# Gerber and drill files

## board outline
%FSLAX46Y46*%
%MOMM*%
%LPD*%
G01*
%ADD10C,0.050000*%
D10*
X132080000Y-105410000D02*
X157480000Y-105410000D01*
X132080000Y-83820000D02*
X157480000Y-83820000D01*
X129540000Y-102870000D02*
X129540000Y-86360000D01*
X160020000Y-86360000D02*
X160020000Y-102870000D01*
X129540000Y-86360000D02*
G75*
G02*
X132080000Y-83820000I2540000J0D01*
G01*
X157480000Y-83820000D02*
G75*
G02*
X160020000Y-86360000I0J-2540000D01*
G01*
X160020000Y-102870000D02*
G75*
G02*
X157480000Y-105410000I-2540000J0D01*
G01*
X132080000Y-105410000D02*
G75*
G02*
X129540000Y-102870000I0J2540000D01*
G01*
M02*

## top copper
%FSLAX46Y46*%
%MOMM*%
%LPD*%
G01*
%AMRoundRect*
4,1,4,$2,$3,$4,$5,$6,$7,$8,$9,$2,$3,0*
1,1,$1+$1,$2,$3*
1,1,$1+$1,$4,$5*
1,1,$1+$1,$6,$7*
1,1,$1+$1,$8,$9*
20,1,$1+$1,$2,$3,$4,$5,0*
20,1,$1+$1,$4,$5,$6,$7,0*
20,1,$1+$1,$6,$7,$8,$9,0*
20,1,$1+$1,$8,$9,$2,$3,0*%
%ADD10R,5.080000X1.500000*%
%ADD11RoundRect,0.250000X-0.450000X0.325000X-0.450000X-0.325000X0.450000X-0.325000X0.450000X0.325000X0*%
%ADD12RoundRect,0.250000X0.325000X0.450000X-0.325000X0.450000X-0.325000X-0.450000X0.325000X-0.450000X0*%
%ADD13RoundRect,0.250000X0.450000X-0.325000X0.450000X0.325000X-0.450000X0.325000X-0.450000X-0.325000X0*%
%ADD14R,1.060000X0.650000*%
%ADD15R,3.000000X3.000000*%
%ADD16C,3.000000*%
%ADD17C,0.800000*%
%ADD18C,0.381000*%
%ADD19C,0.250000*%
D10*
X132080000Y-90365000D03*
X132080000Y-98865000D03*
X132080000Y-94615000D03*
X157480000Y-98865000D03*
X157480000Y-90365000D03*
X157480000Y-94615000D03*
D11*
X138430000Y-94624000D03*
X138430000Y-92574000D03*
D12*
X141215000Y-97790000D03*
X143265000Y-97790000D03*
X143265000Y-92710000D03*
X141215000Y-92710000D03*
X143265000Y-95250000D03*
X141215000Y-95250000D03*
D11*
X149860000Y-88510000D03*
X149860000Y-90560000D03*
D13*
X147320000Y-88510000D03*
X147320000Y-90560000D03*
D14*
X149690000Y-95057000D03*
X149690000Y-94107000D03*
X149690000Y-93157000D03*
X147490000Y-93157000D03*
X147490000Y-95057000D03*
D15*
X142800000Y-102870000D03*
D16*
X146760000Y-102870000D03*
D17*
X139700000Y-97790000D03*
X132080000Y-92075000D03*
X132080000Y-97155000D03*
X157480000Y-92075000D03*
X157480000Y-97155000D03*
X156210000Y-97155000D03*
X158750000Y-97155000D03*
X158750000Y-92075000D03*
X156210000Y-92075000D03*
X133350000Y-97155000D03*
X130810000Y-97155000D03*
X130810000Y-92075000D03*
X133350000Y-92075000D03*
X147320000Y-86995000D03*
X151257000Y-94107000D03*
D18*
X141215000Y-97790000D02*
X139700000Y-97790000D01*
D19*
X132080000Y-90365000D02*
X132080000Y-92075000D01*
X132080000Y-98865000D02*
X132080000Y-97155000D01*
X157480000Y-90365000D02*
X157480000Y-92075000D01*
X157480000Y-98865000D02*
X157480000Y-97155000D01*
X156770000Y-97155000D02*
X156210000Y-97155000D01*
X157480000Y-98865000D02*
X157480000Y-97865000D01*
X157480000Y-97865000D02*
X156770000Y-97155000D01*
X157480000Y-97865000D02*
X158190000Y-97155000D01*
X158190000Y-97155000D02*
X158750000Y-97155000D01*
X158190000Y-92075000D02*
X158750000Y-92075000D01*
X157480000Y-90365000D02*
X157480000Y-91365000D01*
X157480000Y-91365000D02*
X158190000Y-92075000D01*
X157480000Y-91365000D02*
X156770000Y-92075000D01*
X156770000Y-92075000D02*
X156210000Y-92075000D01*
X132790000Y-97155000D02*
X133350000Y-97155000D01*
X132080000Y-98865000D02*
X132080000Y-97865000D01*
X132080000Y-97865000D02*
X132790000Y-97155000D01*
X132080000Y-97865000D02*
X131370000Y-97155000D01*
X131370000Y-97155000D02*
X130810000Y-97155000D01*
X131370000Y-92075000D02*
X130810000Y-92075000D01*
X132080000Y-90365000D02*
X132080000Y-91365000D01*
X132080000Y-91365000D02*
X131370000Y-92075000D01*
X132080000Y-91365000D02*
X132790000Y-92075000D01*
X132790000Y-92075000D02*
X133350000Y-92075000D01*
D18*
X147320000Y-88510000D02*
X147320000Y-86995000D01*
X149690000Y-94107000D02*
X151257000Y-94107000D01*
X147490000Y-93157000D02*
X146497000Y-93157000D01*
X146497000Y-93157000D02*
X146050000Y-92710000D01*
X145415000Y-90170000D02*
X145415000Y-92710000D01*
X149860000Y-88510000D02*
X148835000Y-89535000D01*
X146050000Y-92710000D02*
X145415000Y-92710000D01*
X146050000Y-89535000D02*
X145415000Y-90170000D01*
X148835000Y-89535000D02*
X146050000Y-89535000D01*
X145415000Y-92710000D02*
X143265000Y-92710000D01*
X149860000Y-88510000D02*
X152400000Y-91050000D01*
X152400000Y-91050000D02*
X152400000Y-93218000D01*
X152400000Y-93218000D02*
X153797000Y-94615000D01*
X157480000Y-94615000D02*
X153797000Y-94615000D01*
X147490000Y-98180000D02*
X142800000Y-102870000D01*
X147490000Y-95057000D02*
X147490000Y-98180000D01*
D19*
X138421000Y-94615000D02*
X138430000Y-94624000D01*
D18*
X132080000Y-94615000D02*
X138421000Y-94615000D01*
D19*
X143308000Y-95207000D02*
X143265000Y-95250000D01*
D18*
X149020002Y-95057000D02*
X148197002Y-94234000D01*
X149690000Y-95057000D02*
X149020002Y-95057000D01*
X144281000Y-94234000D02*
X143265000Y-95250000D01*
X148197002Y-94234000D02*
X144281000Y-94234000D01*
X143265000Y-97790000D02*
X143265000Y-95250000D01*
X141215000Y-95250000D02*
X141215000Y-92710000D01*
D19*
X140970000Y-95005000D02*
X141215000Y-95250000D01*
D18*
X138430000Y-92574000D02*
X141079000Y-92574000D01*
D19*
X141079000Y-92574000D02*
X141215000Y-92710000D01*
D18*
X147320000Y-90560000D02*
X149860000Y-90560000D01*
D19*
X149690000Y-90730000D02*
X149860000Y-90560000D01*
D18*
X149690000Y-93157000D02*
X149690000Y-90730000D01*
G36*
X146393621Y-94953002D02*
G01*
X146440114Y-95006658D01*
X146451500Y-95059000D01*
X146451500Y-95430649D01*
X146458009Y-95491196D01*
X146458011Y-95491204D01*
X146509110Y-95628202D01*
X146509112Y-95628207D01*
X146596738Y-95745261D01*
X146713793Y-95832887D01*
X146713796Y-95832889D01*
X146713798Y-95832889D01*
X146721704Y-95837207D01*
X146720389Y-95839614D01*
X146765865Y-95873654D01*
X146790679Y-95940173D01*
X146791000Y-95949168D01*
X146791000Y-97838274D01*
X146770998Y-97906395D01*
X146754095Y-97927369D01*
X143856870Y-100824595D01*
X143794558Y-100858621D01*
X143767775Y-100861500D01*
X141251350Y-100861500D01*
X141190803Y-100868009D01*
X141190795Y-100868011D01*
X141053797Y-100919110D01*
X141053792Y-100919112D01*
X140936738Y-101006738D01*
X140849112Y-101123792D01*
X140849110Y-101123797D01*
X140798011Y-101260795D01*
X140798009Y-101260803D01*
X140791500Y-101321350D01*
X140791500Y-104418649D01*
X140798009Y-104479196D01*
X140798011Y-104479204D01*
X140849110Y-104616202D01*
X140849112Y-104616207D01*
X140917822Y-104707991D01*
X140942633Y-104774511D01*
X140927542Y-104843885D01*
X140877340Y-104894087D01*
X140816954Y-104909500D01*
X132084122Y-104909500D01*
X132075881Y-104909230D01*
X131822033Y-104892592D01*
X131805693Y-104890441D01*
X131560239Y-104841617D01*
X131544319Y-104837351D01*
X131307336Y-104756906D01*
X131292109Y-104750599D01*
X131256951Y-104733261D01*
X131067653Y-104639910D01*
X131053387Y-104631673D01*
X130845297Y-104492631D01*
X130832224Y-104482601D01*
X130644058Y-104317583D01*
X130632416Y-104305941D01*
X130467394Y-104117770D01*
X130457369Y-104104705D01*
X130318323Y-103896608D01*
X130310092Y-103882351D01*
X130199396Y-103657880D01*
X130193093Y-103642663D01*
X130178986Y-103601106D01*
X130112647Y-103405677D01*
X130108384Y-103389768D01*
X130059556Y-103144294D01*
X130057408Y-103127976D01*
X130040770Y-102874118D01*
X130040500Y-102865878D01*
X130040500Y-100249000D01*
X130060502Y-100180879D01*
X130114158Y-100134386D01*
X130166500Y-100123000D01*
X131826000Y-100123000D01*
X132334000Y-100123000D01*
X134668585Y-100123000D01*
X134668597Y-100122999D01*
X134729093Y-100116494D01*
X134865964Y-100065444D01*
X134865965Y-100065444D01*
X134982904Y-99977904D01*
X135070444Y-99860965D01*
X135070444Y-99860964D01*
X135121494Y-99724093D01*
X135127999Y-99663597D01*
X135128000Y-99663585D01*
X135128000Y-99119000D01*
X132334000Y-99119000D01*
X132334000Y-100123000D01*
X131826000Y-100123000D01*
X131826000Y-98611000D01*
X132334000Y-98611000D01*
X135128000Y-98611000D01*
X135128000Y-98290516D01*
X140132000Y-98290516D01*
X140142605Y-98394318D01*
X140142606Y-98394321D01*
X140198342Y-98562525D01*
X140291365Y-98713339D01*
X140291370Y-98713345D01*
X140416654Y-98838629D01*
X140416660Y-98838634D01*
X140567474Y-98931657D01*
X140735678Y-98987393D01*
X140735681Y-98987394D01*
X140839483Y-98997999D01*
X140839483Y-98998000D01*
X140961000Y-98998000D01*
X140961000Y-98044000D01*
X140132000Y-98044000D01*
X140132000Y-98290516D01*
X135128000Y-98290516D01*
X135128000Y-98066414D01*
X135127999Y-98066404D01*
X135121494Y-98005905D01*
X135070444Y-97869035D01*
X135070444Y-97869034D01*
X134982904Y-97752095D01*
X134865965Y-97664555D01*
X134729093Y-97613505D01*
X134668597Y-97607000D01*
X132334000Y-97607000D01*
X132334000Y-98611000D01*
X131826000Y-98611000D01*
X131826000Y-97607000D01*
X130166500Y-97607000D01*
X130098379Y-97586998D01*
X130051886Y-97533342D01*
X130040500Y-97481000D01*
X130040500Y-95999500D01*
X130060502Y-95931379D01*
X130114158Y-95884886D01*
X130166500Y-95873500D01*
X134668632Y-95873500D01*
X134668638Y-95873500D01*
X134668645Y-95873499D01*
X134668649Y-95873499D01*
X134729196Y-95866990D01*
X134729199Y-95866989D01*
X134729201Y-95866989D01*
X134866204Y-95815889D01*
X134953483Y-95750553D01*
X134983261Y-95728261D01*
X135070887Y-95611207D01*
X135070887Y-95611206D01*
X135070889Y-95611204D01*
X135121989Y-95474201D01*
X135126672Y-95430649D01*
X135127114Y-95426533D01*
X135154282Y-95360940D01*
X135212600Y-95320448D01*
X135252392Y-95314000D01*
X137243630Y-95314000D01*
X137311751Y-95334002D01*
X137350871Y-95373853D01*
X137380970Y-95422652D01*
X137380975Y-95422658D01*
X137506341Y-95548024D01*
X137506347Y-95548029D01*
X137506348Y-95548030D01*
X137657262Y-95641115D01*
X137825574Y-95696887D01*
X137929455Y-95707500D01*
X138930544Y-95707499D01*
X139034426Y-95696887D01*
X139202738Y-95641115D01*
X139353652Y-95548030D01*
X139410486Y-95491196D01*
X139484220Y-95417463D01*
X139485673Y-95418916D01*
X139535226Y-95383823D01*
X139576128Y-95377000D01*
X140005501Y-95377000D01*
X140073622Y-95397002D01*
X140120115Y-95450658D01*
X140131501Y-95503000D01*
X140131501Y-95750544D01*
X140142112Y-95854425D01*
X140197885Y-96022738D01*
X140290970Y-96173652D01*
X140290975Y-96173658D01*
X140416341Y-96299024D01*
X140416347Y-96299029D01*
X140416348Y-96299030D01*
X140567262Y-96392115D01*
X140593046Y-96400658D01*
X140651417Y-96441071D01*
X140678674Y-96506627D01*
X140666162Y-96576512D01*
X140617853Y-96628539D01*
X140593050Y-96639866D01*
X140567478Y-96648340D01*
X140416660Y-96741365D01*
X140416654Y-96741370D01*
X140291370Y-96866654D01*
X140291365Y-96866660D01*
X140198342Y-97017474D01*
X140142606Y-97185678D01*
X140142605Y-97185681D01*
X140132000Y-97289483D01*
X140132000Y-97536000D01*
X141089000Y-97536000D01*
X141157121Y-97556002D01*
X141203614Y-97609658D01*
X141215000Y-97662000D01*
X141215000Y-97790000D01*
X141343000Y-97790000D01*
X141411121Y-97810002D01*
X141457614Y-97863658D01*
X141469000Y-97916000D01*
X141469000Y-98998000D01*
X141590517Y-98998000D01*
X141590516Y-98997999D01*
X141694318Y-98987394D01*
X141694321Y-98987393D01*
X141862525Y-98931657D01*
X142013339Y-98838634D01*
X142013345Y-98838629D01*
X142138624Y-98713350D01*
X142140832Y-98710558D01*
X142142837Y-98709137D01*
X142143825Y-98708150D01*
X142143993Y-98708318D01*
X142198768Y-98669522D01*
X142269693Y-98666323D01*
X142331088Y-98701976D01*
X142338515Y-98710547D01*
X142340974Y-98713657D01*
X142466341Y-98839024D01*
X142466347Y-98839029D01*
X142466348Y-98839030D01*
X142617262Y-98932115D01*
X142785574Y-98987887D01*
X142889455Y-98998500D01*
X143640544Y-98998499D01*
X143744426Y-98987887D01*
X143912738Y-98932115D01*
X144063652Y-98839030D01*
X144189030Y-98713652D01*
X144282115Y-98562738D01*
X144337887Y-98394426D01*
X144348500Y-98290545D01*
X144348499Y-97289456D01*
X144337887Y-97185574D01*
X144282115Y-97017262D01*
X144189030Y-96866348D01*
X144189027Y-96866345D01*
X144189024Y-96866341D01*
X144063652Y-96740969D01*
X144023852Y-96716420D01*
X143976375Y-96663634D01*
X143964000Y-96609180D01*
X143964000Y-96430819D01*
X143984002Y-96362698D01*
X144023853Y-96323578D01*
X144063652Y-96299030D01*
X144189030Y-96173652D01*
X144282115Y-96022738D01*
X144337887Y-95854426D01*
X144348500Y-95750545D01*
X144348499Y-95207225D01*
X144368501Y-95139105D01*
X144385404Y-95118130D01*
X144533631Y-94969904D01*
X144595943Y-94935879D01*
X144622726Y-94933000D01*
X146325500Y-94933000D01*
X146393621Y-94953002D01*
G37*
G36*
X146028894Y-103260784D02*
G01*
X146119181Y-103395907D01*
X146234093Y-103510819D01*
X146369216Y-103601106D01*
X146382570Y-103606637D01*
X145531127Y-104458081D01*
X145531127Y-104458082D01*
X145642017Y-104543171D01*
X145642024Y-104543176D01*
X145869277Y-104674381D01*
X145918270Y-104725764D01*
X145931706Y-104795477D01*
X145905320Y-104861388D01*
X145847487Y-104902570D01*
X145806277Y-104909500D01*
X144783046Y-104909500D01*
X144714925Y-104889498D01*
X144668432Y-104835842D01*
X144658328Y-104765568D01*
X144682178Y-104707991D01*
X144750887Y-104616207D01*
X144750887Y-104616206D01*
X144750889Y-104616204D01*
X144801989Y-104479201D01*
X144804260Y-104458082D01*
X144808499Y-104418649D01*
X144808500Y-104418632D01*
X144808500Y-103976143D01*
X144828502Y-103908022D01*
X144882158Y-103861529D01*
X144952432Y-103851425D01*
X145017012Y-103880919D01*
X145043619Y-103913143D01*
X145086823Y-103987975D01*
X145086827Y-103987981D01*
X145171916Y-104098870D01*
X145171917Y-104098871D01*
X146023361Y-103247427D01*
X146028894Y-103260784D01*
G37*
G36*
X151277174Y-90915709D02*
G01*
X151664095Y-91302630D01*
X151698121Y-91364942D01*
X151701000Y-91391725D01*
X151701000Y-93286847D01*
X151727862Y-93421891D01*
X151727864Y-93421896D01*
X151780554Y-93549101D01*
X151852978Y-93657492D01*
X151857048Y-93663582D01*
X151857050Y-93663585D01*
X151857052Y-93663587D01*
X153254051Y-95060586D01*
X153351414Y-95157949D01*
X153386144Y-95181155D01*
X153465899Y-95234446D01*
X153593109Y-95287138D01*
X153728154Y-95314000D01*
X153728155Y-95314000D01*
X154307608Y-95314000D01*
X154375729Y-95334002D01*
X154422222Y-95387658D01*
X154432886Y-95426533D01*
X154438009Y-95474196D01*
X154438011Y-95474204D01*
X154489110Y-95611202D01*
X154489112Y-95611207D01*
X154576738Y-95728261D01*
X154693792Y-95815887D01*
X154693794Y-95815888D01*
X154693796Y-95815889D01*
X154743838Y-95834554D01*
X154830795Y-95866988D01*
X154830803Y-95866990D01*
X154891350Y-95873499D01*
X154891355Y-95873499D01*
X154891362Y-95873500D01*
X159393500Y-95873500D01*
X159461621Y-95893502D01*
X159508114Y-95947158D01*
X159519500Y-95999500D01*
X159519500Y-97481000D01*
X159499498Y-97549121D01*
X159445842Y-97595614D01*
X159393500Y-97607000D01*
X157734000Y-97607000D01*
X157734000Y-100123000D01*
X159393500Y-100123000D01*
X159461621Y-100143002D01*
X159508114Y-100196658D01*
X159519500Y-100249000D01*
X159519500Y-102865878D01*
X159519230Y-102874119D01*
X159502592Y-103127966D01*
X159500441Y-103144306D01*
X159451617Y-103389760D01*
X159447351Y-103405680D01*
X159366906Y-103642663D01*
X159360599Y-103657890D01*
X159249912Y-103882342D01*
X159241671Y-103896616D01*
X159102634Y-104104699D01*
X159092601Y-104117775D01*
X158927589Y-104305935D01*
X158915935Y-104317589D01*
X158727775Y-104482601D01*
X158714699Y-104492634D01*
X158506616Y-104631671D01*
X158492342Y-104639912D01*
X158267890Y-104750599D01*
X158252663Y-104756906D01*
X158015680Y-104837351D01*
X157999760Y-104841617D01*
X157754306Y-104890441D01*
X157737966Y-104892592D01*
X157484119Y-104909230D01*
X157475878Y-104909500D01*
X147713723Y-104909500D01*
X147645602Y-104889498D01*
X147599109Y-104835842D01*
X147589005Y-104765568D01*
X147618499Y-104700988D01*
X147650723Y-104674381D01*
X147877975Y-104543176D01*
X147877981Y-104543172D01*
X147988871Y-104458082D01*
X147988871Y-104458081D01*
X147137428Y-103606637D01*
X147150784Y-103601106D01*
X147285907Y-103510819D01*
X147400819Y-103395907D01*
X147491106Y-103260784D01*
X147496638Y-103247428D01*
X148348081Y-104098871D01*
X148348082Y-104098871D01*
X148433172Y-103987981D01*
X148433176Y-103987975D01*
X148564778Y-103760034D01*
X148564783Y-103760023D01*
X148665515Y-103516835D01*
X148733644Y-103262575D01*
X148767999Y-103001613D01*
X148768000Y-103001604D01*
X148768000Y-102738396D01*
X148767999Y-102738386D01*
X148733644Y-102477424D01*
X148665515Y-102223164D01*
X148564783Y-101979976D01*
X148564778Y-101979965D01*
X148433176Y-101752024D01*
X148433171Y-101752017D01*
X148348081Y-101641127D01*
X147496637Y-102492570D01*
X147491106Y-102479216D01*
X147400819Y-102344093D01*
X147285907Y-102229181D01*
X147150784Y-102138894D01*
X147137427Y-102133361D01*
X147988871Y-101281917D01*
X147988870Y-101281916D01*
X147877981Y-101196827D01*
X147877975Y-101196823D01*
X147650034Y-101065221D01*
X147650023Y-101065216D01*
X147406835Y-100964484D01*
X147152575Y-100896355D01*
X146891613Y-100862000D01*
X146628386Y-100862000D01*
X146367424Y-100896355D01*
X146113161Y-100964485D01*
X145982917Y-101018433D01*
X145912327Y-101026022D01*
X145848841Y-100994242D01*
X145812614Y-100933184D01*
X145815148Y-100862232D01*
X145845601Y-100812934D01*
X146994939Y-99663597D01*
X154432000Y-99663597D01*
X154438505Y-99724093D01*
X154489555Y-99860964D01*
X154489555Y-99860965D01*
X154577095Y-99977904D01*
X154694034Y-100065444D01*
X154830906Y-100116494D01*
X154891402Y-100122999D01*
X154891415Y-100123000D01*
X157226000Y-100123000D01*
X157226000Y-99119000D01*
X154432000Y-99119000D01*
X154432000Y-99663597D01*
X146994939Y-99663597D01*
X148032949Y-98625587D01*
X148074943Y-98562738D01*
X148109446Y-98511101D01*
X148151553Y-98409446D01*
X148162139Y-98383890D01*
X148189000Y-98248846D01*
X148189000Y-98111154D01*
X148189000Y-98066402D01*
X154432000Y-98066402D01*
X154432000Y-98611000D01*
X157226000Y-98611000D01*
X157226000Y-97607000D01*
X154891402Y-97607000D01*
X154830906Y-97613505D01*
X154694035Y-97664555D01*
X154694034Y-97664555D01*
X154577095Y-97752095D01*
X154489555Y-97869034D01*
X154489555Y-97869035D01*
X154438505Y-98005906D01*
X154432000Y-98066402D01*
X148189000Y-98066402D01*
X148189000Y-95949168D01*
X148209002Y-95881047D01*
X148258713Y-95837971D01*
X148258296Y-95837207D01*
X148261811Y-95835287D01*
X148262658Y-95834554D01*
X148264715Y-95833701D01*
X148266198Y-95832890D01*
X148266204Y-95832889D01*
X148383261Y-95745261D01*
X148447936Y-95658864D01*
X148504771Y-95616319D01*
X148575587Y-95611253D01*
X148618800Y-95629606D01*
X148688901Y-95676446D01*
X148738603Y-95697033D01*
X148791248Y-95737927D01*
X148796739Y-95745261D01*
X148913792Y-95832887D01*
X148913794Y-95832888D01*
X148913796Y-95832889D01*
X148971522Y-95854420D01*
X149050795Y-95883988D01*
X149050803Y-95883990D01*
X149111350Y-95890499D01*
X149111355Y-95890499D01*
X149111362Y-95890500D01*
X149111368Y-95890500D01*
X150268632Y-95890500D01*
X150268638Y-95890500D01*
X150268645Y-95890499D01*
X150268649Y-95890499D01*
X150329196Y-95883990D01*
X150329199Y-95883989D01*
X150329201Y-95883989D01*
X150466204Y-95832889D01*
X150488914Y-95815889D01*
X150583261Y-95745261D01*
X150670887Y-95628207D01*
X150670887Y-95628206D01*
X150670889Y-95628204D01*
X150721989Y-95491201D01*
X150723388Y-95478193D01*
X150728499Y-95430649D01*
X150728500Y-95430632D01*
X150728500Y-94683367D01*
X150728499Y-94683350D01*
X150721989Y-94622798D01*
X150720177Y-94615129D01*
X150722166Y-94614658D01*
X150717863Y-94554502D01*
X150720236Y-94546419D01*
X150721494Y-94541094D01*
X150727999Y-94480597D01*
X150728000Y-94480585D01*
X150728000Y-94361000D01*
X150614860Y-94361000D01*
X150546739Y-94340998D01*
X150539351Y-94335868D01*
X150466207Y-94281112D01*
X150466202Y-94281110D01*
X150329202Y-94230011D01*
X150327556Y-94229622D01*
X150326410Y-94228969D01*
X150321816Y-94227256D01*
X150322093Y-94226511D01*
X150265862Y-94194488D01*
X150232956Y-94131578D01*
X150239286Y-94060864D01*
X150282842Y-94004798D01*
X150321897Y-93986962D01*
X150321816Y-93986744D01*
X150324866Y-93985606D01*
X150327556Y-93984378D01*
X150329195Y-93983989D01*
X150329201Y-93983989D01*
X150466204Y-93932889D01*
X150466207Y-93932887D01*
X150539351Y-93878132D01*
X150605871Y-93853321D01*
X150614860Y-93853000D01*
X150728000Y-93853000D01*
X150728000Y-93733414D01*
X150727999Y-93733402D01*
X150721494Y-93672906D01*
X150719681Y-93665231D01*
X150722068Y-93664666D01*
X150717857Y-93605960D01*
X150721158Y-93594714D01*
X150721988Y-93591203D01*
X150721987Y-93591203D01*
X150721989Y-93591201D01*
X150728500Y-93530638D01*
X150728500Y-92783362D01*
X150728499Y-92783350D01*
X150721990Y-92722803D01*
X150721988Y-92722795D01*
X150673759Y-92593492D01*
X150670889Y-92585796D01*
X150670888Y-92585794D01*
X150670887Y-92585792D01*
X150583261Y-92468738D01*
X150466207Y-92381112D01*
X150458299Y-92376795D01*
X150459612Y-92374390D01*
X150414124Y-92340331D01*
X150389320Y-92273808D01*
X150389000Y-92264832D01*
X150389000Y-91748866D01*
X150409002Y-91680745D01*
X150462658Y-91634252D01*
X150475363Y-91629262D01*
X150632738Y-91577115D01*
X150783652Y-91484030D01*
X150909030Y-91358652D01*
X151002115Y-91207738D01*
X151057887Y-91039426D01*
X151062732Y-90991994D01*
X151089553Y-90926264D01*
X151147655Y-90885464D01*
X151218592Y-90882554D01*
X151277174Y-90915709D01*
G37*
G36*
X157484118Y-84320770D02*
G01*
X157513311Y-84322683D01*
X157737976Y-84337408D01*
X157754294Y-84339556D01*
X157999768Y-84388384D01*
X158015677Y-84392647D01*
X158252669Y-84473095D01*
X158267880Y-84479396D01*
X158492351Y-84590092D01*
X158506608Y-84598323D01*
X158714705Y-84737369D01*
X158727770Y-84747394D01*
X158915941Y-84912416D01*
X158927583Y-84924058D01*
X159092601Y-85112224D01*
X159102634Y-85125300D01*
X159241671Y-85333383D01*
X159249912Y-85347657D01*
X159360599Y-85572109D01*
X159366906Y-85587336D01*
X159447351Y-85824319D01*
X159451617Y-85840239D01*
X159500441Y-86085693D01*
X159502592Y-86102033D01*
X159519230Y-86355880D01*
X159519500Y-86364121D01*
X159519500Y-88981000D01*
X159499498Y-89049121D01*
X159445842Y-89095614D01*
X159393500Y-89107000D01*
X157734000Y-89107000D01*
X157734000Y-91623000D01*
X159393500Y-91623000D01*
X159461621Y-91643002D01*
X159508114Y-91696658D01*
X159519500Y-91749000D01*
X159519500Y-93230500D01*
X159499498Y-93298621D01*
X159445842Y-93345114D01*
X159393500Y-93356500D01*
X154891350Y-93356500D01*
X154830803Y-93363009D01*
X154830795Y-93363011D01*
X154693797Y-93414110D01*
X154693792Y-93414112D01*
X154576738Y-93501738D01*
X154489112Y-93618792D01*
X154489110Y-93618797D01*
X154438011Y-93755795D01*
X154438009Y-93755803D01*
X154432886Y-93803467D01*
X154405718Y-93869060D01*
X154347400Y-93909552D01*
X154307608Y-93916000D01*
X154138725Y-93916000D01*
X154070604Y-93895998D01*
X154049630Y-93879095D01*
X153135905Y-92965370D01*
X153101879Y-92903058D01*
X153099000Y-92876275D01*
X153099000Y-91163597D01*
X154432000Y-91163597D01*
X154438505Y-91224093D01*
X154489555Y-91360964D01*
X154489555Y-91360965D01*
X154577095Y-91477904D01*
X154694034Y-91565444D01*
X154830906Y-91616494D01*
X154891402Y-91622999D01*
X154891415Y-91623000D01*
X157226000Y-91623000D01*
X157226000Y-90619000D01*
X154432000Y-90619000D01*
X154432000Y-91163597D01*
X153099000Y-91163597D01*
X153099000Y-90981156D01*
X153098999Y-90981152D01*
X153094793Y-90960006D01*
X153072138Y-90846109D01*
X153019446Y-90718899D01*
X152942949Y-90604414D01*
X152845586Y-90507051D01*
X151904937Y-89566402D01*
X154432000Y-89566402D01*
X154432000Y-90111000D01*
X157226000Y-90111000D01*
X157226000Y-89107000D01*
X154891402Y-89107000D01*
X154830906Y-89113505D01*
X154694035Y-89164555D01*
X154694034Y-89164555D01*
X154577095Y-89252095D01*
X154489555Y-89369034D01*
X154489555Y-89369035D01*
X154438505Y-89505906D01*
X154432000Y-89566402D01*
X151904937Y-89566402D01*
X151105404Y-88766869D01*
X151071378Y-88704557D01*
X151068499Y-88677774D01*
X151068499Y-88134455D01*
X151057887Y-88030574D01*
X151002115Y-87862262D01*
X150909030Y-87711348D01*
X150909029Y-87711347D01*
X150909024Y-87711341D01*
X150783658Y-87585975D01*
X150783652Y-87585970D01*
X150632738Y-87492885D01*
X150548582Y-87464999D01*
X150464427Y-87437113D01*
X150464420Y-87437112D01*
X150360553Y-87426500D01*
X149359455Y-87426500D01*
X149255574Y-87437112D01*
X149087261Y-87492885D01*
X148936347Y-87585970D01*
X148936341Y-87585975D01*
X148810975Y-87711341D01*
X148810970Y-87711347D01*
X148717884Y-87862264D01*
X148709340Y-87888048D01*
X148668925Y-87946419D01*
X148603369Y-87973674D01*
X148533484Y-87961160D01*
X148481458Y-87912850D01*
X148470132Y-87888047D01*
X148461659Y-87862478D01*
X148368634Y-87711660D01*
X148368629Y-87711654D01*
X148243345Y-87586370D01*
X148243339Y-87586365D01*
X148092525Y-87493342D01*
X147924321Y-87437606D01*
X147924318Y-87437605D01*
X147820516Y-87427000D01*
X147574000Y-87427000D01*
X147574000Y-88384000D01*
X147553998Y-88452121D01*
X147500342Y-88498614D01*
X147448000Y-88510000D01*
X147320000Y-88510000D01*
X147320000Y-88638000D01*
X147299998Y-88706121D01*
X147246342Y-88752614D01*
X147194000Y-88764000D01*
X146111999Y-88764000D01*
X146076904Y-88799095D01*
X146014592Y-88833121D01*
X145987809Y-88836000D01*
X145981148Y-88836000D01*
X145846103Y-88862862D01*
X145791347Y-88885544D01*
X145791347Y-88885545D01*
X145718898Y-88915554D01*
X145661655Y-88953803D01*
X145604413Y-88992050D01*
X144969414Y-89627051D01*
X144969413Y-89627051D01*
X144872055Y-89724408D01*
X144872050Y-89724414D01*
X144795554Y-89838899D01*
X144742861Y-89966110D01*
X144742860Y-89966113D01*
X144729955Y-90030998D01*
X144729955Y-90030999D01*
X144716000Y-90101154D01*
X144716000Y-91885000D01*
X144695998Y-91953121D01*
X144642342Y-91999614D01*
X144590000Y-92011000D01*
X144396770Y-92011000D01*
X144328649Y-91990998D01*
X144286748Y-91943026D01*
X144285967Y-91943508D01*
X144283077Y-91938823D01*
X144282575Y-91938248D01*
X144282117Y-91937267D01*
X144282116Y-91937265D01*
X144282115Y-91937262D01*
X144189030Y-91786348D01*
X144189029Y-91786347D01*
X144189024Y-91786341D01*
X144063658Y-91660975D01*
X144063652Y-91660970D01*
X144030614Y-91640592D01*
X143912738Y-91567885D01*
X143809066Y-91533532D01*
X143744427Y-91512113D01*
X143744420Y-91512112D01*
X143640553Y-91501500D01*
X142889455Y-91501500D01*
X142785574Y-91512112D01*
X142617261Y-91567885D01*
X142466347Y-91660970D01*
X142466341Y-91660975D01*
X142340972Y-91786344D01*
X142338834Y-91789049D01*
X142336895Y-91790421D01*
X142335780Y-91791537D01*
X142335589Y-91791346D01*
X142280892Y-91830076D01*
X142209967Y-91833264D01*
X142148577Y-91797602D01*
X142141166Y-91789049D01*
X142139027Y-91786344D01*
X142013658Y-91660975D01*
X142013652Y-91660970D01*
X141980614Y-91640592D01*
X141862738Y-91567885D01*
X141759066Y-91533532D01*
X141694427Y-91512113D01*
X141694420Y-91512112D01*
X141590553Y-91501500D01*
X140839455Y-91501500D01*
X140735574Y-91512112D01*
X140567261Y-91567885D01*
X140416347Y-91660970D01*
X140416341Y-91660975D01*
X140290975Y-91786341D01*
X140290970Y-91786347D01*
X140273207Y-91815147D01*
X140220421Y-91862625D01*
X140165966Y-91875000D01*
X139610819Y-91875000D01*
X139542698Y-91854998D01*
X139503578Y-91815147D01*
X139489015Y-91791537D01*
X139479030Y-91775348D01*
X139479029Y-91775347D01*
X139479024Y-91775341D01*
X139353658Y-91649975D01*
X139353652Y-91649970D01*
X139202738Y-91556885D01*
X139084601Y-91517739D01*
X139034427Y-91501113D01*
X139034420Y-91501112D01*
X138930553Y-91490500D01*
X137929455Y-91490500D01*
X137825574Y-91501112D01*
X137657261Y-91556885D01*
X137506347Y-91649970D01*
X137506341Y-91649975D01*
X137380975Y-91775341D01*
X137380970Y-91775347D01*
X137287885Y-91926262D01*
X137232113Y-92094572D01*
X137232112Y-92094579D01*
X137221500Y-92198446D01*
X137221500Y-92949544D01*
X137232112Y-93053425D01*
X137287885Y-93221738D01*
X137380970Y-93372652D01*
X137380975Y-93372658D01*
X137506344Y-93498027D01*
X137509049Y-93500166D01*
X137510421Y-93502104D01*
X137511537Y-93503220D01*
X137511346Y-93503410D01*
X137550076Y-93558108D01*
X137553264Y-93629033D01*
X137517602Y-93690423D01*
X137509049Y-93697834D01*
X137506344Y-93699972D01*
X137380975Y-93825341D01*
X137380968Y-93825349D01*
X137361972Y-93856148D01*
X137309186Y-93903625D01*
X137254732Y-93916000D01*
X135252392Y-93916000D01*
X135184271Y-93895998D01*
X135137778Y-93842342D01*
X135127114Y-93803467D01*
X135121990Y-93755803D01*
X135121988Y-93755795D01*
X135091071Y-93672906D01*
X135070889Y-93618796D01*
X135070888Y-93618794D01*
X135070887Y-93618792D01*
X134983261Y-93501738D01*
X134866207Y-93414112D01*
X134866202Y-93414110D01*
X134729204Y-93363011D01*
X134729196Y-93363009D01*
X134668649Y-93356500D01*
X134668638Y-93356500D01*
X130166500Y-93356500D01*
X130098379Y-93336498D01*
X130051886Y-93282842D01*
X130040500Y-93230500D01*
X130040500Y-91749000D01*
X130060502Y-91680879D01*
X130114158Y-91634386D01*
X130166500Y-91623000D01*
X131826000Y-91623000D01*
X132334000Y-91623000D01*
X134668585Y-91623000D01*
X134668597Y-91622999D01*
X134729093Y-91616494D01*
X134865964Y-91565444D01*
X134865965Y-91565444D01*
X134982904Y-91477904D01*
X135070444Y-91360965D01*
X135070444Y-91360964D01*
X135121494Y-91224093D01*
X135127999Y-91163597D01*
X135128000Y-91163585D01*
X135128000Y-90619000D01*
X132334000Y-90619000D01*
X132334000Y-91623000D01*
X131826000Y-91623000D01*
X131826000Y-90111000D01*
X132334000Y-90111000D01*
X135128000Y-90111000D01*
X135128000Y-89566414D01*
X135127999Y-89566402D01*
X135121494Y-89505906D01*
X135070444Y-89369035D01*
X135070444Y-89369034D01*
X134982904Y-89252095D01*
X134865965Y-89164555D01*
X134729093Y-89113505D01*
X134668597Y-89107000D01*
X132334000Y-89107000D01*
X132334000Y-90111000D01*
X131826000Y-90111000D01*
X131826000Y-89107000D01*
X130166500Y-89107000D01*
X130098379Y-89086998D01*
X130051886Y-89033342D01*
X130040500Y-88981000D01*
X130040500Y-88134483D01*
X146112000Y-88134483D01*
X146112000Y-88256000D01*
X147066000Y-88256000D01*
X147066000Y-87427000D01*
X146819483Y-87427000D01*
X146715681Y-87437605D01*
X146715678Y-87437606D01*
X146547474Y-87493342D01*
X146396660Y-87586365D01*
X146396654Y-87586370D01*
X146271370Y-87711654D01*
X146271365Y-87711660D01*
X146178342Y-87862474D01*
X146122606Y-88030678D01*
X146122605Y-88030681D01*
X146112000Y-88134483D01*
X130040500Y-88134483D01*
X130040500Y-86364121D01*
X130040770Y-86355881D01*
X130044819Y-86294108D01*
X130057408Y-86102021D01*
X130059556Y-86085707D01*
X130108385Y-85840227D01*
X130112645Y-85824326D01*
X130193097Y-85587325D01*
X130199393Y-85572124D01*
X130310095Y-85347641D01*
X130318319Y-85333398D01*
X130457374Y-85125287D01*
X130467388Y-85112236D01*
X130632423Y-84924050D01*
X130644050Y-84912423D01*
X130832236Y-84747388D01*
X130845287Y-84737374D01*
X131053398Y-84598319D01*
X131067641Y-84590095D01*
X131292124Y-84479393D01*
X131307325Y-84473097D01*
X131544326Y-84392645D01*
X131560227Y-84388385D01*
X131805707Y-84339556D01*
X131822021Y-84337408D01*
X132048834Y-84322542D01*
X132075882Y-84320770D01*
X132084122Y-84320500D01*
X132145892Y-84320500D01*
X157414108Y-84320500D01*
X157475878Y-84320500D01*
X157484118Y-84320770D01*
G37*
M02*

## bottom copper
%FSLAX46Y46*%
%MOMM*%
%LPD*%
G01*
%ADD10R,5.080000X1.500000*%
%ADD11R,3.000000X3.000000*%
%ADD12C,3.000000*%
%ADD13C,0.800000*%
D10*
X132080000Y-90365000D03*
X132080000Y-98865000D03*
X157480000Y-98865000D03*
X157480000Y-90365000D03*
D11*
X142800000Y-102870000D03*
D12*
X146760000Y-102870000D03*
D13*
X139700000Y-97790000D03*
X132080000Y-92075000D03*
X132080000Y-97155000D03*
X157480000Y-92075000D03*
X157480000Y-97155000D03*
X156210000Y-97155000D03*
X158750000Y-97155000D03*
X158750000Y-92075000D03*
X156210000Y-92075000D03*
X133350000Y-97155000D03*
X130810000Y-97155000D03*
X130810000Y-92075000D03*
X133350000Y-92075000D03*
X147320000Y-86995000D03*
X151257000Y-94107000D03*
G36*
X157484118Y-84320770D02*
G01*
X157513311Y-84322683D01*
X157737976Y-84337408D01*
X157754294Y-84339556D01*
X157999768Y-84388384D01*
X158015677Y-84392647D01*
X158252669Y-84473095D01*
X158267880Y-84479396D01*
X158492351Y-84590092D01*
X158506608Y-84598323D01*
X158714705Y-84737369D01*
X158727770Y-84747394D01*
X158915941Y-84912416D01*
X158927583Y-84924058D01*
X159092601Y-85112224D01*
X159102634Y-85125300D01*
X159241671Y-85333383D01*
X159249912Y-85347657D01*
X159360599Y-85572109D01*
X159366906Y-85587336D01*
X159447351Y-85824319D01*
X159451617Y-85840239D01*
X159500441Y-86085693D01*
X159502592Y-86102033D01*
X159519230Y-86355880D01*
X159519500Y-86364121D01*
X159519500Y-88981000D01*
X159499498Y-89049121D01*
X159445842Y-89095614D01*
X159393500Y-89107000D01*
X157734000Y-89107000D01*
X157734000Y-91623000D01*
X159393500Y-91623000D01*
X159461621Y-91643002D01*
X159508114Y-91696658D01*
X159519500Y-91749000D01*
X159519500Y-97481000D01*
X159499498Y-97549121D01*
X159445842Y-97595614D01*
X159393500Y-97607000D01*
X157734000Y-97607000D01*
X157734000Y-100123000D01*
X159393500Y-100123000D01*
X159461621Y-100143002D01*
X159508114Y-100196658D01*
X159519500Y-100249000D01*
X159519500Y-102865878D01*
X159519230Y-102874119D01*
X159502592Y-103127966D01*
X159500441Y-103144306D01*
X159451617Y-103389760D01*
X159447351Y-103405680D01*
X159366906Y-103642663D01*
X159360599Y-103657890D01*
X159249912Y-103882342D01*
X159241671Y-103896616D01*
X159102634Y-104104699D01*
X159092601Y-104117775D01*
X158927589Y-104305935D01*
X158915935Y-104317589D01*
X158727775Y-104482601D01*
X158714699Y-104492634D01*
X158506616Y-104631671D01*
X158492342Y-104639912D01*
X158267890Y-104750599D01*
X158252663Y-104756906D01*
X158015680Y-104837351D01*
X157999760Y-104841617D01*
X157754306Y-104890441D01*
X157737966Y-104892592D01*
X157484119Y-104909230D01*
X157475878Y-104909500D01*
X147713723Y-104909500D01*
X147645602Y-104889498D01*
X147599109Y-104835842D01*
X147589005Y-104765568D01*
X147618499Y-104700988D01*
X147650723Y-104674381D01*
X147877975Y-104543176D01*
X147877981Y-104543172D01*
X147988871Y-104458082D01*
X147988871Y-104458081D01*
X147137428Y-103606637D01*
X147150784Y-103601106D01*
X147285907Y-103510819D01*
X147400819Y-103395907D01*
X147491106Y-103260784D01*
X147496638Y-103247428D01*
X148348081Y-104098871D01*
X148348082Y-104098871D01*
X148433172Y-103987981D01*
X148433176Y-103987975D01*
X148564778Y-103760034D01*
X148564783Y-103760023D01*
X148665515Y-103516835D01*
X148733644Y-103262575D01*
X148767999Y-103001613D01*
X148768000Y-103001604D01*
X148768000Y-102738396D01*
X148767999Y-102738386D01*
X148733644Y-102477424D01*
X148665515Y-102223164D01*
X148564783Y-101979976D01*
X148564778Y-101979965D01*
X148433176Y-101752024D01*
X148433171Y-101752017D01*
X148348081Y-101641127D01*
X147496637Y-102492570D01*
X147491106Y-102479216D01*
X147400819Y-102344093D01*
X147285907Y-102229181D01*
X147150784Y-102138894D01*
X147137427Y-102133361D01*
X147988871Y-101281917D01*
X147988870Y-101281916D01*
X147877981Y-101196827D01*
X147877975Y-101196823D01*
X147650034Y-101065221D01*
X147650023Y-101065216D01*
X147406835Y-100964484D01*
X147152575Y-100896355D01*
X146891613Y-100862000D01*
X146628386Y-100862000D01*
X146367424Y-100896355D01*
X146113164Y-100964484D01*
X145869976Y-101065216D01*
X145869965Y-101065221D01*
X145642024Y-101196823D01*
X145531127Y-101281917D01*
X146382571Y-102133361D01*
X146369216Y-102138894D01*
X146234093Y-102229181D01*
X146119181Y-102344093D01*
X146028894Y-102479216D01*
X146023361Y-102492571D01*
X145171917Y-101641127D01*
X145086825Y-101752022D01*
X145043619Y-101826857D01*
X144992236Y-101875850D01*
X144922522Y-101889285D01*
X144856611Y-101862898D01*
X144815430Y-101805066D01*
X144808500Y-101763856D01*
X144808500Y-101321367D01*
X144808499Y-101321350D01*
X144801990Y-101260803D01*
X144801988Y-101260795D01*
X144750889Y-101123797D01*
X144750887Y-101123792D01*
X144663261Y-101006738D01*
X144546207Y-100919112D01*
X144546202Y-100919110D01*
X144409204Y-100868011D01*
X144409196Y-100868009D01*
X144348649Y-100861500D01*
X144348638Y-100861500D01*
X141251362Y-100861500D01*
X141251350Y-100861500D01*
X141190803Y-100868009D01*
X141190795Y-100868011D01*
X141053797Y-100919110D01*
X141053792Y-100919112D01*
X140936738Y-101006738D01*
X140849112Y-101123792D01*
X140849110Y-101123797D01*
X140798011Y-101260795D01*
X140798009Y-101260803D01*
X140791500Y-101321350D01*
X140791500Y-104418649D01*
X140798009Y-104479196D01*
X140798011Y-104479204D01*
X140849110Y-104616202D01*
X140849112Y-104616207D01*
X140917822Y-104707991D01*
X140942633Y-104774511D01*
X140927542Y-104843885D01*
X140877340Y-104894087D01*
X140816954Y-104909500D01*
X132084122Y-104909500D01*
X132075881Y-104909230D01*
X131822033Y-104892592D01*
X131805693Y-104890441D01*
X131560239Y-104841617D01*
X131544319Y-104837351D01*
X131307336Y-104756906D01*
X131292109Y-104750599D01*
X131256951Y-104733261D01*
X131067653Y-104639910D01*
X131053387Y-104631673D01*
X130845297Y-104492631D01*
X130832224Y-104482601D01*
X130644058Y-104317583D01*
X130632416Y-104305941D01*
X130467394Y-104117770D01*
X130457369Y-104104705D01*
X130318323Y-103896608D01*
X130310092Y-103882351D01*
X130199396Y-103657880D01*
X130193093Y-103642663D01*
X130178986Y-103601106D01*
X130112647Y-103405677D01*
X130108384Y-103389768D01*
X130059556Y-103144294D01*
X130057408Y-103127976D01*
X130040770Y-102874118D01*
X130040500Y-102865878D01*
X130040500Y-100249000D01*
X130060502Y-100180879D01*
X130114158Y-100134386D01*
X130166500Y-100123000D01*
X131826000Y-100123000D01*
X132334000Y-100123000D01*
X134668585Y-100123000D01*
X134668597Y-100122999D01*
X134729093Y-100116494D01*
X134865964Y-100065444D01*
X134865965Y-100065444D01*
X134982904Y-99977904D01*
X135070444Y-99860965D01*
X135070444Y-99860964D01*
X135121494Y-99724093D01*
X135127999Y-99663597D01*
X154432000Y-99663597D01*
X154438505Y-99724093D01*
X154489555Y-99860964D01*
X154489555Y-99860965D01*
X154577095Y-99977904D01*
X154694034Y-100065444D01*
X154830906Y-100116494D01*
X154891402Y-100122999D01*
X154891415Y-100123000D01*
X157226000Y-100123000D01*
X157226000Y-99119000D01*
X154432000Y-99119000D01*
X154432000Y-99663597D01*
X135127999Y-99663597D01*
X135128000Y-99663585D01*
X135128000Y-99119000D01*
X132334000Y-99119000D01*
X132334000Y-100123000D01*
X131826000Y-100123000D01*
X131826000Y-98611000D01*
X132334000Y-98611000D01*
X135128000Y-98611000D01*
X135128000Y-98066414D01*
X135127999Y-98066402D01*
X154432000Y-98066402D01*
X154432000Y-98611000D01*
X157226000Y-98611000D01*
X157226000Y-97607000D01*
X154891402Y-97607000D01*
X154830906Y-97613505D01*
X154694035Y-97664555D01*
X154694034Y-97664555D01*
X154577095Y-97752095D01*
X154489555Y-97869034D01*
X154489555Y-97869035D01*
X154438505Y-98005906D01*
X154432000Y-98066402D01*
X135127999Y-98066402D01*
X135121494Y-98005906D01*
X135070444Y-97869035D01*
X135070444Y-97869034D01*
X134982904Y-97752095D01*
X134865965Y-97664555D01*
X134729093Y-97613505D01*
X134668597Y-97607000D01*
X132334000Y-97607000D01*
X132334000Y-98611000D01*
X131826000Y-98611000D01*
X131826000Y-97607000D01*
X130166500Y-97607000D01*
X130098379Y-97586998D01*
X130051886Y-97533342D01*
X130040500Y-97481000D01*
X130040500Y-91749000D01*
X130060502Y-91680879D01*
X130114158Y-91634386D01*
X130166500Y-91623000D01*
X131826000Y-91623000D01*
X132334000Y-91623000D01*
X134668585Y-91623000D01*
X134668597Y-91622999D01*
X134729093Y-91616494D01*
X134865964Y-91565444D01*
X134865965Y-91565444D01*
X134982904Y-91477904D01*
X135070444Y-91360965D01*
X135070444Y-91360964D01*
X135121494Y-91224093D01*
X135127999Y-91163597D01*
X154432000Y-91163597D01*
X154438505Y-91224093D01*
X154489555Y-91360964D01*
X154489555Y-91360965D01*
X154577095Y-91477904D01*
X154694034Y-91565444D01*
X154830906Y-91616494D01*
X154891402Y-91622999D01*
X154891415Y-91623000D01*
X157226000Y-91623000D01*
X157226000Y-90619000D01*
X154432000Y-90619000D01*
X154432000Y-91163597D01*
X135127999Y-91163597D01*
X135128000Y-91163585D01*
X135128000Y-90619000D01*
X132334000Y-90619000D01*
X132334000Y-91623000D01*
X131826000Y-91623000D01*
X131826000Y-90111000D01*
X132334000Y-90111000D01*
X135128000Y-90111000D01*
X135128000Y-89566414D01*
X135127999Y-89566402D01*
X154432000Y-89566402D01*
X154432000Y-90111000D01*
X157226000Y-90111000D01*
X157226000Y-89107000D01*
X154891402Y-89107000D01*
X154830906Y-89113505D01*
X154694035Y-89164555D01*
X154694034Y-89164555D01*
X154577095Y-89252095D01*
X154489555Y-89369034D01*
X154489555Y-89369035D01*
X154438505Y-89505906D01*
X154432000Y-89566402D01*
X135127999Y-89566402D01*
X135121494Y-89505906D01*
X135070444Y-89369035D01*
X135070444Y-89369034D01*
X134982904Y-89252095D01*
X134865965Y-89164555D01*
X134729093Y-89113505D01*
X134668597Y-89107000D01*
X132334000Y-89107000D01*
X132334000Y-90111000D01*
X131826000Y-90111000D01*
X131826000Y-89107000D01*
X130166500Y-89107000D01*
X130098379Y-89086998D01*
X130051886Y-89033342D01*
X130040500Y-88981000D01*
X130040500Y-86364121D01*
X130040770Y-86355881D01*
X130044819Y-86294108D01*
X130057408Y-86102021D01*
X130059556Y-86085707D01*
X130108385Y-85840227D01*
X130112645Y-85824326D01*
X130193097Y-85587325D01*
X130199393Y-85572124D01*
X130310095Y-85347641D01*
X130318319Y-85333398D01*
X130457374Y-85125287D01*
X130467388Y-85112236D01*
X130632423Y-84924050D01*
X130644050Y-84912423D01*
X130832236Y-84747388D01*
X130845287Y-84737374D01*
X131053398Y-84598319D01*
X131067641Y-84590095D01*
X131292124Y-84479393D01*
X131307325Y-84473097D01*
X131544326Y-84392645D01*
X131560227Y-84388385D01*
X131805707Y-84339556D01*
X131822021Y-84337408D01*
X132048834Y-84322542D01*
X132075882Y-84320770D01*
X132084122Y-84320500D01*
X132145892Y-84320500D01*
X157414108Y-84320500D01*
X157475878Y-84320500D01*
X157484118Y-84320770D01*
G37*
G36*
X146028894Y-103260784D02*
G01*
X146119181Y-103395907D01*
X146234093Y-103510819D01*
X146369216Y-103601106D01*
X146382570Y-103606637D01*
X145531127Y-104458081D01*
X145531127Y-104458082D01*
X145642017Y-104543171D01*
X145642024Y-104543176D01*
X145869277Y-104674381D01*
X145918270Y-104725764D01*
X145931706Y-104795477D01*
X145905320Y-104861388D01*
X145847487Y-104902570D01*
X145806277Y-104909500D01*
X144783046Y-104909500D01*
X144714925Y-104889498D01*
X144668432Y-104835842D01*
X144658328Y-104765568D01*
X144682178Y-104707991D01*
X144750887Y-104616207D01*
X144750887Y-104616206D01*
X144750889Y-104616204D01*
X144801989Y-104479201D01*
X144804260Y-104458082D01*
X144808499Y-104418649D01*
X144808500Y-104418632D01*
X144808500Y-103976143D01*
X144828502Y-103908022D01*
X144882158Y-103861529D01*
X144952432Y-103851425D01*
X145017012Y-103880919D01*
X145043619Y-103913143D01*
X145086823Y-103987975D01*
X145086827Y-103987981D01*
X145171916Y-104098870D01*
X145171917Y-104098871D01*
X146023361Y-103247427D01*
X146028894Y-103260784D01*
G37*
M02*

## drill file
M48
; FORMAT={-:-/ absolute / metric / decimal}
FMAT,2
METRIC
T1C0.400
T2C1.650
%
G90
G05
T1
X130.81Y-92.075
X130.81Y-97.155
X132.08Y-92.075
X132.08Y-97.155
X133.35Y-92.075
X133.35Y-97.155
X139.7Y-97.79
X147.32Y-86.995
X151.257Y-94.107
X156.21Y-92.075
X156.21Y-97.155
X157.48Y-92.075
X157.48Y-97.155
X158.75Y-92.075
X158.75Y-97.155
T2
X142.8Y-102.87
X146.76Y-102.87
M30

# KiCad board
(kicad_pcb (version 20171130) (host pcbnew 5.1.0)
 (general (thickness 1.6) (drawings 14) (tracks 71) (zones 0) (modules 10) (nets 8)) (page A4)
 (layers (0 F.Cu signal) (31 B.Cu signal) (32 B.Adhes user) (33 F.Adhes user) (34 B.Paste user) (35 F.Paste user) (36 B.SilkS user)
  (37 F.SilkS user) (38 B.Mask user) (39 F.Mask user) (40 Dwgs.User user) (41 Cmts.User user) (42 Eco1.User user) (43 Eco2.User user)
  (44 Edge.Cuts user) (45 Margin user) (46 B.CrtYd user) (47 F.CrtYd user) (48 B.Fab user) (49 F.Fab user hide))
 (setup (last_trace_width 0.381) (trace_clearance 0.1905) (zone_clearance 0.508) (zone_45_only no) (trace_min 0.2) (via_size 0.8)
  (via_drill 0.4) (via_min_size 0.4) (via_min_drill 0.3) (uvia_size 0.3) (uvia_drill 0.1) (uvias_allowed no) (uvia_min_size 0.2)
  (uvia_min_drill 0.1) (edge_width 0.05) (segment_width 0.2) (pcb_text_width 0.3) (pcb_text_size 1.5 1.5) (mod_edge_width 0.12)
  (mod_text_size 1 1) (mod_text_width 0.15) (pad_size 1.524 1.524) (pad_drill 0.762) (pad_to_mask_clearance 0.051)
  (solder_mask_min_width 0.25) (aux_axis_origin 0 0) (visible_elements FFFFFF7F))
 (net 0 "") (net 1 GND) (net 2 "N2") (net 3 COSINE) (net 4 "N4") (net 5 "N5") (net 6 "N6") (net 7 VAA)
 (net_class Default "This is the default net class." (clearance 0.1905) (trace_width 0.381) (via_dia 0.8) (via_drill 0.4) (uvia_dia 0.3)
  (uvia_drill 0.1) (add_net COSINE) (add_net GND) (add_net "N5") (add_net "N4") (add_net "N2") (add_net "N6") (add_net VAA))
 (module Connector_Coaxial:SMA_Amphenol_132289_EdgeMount (layer F.Cu) (at 132.08 94.615 180)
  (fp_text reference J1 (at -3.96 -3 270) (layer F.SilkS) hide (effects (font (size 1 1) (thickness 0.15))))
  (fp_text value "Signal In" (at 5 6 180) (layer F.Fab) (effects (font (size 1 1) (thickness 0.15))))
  (pad 2 smd rect (at 0 4.25 270) (size 1.5 5.08) (layers B.Cu B.Paste B.Mask) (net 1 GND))
  (pad 2 smd rect (at 0 -4.25 270) (size 1.5 5.08) (layers B.Cu B.Paste B.Mask) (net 1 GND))
  (pad 2 smd rect (at 0 4.25 270) (size 1.5 5.08) (layers F.Cu F.Paste F.Mask) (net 1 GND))
  (pad 2 smd rect (at 0 -4.25 270) (size 1.5 5.08) (layers F.Cu F.Paste F.Mask) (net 1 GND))
  (pad 1 smd rect (at 0 0 270) (size 1.5 5.08) (layers F.Cu F.Paste F.Mask) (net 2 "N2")))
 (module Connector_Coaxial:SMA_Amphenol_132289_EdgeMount (layer F.Cu) (at 157.48 94.615)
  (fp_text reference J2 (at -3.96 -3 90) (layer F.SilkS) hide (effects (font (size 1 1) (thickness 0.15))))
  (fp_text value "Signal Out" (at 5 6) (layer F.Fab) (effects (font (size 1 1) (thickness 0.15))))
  (pad 2 smd rect (at 0 4.25 90) (size 1.5 5.08) (layers B.Cu B.Paste B.Mask) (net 1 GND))
  (pad 2 smd rect (at 0 -4.25 90) (size 1.5 5.08) (layers B.Cu B.Paste B.Mask) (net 1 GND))
  (pad 2 smd rect (at 0 4.25 90) (size 1.5 5.08) (layers F.Cu F.Paste F.Mask) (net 1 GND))
  (pad 2 smd rect (at 0 -4.25 90) (size 1.5 5.08) (layers F.Cu F.Paste F.Mask) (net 1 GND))
  (pad 1 smd rect (at 0 0 90) (size 1.5 5.08) (layers F.Cu F.Paste F.Mask) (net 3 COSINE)))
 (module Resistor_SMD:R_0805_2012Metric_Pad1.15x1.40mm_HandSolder (layer F.Cu) (at 138.43 93.599 270)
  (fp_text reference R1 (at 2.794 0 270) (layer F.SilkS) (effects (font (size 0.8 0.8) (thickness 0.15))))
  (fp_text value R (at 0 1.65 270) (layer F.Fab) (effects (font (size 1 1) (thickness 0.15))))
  (pad 2 smd roundrect (at 1.025 0 270) (size 1.15 1.4) (layers F.Cu F.Paste F.Mask) (roundrect_rratio 0.217391) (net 2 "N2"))
  (pad 1 smd roundrect (at -1.025 0 270) (size 1.15 1.4) (layers F.Cu F.Paste F.Mask) (roundrect_rratio 0.217391) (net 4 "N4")))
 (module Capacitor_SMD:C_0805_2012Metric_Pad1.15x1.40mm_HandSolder (layer F.Cu) (at 142.24 97.79 180)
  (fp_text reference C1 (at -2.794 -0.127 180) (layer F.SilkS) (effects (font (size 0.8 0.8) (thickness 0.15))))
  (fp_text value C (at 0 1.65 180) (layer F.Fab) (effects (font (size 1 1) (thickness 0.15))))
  (pad 2 smd roundrect (at 1.025 0 180) (size 1.15 1.4) (layers F.Cu F.Paste F.Mask) (roundrect_rratio 0.217391) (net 1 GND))
  (pad 1 smd roundrect (at -1.025 0 180) (size 1.15 1.4) (layers F.Cu F.Paste F.Mask) (roundrect_rratio 0.217391) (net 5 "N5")))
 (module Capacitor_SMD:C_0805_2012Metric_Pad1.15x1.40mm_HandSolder (layer F.Cu) (at 142.24 92.71 180)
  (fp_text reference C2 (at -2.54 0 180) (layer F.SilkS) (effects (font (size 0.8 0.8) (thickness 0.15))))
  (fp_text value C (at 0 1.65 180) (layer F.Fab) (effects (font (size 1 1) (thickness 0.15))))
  (pad 1 smd roundrect (at -1.025 0 180) (size 1.15 1.4) (layers F.Cu F.Paste F.Mask) (roundrect_rratio 0.217391) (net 3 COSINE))
  (pad 2 smd roundrect (at 1.025 0 180) (size 1.15 1.4) (layers F.Cu F.Paste F.Mask) (roundrect_rratio 0.217391) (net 4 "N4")))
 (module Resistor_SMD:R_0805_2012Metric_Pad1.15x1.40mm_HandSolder (layer F.Cu) (at 142.24 95.25 180)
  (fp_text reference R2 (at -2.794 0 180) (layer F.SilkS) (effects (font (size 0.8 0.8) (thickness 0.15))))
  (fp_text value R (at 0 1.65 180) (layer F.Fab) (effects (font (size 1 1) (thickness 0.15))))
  (pad 1 smd roundrect (at -1.025 0 180) (size 1.15 1.4) (layers F.Cu F.Paste F.Mask) (roundrect_rratio 0.217391) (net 5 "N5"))
  (pad 2 smd roundrect (at 1.025 0 180) (size 1.15 1.4) (layers F.Cu F.Paste F.Mask) (roundrect_rratio 0.217391) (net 4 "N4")))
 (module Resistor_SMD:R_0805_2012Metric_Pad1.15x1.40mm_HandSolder (layer F.Cu) (at 149.86 89.535 270)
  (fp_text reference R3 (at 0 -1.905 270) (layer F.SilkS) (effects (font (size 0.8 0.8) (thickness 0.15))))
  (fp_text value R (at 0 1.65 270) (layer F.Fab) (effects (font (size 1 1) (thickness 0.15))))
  (pad 1 smd roundrect (at -1.025 0 270) (size 1.15 1.4) (layers F.Cu F.Paste F.Mask) (roundrect_rratio 0.217391) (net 3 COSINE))
  (pad 2 smd roundrect (at 1.025 0 270) (size 1.15 1.4) (layers F.Cu F.Paste F.Mask) (roundrect_rratio 0.217391) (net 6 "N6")))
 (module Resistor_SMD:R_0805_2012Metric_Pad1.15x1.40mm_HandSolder (layer F.Cu) (at 147.32 89.535 90)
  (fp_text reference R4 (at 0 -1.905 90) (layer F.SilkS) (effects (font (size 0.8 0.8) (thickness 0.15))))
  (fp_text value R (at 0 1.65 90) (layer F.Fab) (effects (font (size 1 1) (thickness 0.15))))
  (pad 2 smd roundrect (at 1.025 0 90) (size 1.15 1.4) (layers F.Cu F.Paste F.Mask) (roundrect_rratio 0.217391) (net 1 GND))
  (pad 1 smd roundrect (at -1.025 0 90) (size 1.15 1.4) (layers F.Cu F.Paste F.Mask) (roundrect_rratio 0.217391) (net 6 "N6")))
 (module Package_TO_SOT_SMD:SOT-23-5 (layer F.Cu) (at 148.59 94.107 180)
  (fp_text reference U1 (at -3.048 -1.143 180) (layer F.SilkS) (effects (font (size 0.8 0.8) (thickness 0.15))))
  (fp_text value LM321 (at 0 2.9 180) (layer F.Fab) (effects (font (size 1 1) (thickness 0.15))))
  (pad 1 smd rect (at -1.1 -0.95 180) (size 1.06 0.65) (layers F.Cu F.Paste F.Mask) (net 5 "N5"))
  (pad 2 smd rect (at -1.1 0 180) (size 1.06 0.65) (layers F.Cu F.Paste F.Mask) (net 1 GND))
  (pad 3 smd rect (at -1.1 0.95 180) (size 1.06 0.65) (layers F.Cu F.Paste F.Mask) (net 6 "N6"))
  (pad 4 smd rect (at 1.1 0.95 180) (size 1.06 0.65) (layers F.Cu F.Paste F.Mask) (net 3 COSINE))
  (pad 5 smd rect (at 1.1 -0.95 180) (size 1.06 0.65) (layers F.Cu F.Paste F.Mask) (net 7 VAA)))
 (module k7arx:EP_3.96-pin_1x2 (layer F.Cu) (at 144.78 102.87)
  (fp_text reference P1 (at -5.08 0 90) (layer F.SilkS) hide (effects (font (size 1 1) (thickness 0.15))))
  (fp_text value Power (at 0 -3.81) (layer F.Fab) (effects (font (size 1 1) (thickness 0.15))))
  (pad 1 thru_hole rect (at -1.98 0) (size 3 3) (drill 1.65) (layers *.Cu *.Mask) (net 7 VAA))
  (pad 2 thru_hole circle (at 1.98 0) (size 3 3) (drill 1.65) (layers *.Cu *.Mask) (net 1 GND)))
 (gr_line (start 132.08 105.41) (end 157.48 105.41) (layer Edge.Cuts) (width 0.05))
 (gr_line (start 132.08 83.82) (end 157.48 83.82) (layer Edge.Cuts) (width 0.05))
 (gr_line (start 129.54 102.87) (end 129.54 86.36) (layer Edge.Cuts) (width 0.05))
 (gr_line (start 160.02 86.36) (end 160.02 102.87) (layer Edge.Cuts) (width 0.05))
 (gr_arc (start 132.08 86.36) (end 132.08 83.82) (angle -90) (layer Edge.Cuts) (width 0.05))
 (gr_arc (start 157.48 86.36) (end 160.02 86.36) (angle -90) (layer Edge.Cuts) (width 0.05))
 (gr_arc (start 157.48 102.87) (end 157.48 105.41) (angle -90) (layer Edge.Cuts) (width 0.05))
 (gr_arc (start 132.08 102.87) (end 129.54 102.87) (angle -90) (layer Edge.Cuts) (width 0.05))
 (via (at 139.7 97.79) (size 0.8) (drill 0.4) (layers F.Cu B.Cu) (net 1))
 (segment (start 141.215 97.79) (end 139.7 97.79) (width 0.381) (layer F.Cu) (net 1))
 (via (at 132.08 92.075) (size 0.8) (drill 0.4) (layers F.Cu B.Cu) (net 1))
 (segment (start 132.08 90.365) (end 132.08 92.075) (width 0.25) (layer F.Cu) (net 1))
 (via (at 132.08 97.155) (size 0.8) (drill 0.4) (layers F.Cu B.Cu) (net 1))
 (segment (start 132.08 98.865) (end 132.08 97.155) (width 0.25) (layer F.Cu) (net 1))
 (via (at 157.48 92.075) (size 0.8) (drill 0.4) (layers F.Cu B.Cu) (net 1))
 (segment (start 157.48 90.365) (end 157.48 92.075) (width 0.25) (layer F.Cu) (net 1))
 (via (at 157.48 97.155) (size 0.8) (drill 0.4) (layers F.Cu B.Cu) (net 1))
 (segment (start 157.48 98.865) (end 157.48 97.155) (width 0.25) (layer F.Cu) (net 1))
 (via (at 156.21 97.155) (size 0.8) (drill 0.4) (layers F.Cu B.Cu) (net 1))
 (segment (start 156.77 97.155) (end 156.21 97.155) (width 0.25) (layer F.Cu) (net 1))
 (segment (start 157.48 98.865) (end 157.48 97.865) (width 0.25) (layer F.Cu) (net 1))
 (segment (start 157.48 97.865) (end 156.77 97.155) (width 0.25) (layer F.Cu) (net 1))
 (via (at 158.75 97.155) (size 0.8) (drill 0.4) (layers F.Cu B.Cu) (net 1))
 (segment (start 157.48 97.865) (end 158.19 97.155) (width 0.25) (layer F.Cu) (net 1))
 (segment (start 158.19 97.155) (end 158.75 97.155) (width 0.25) (layer F.Cu) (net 1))
 (via (at 158.75 92.075) (size 0.8) (drill 0.4) (layers F.Cu B.Cu) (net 1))
 (segment (start 158.19 92.075) (end 158.75 92.075) (width 0.25) (layer F.Cu) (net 1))
 (segment (start 157.48 90.365) (end 157.48 91.365) (width 0.25) (layer F.Cu) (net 1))
 (segment (start 157.48 91.365) (end 158.19 92.075) (width 0.25) (layer F.Cu) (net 1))
 (via (at 156.21 92.075) (size 0.8) (drill 0.4) (layers F.Cu B.Cu) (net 1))
 (segment (start 157.48 91.365) (end 156.77 92.075) (width 0.25) (layer F.Cu) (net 1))
 (segment (start 156.77 92.075) (end 156.21 92.075) (width 0.25) (layer F.Cu) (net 1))
 (via (at 133.35 97.155) (size 0.8) (drill 0.4) (layers F.Cu B.Cu) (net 1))
 (segment (start 132.79 97.155) (end 133.35 97.155) (width 0.25) (layer F.Cu) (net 1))
 (segment (start 132.08 98.865) (end 132.08 97.865) (width 0.25) (layer F.Cu) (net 1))
 (segment (start 132.08 97.865) (end 132.79 97.155) (width 0.25) (layer F.Cu) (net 1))
 (via (at 130.81 97.155) (size 0.8) (drill 0.4) (layers F.Cu B.Cu) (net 1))
 (segment (start 132.08 97.865) (end 131.37 97.155) (width 0.25) (layer F.Cu) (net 1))
 (segment (start 131.37 97.155) (end 130.81 97.155) (width 0.25) (layer F.Cu) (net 1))
 (via (at 130.81 92.075) (size 0.8) (drill 0.4) (layers F.Cu B.Cu) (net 1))
 (segment (start 131.37 92.075) (end 130.81 92.075) (width 0.25) (layer F.Cu) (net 1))
 (segment (start 132.08 90.365) (end 132.08 91.365) (width 0.25) (layer F.Cu) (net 1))
 (segment (start 132.08 91.365) (end 131.37 92.075) (width 0.25) (layer F.Cu) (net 1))
 (via (at 133.35 92.075) (size 0.8) (drill 0.4) (layers F.Cu B.Cu) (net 1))
 (segment (start 132.08 91.365) (end 132.79 92.075) (width 0.25) (layer F.Cu) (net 1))
 (segment (start 132.79 92.075) (end 133.35 92.075) (width 0.25) (layer F.Cu) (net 1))
 (via (at 147.32 86.995) (size 0.8) (drill 0.4) (layers F.Cu B.Cu) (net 1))
 (segment (start 147.32 88.51) (end 147.32 86.995) (width 0.381) (layer F.Cu) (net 1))
 (via (at 151.257 94.107) (size 0.8) (drill 0.4) (layers F.Cu B.Cu) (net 1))
 (segment (start 149.69 94.107) (end 151.257 94.107) (width 0.381) (layer F.Cu) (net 1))
 (segment (start 147.49 93.157) (end 146.497 93.157) (width 0.381) (layer F.Cu) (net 3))
 (segment (start 146.497 93.157) (end 146.05 92.71) (width 0.381) (layer F.Cu) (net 3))
 (segment (start 145.415 90.17) (end 145.415 92.71) (width 0.381) (layer F.Cu) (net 3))
 (segment (start 149.86 88.51) (end 148.835 89.535) (width 0.381) (layer F.Cu) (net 3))
 (segment (start 146.05 92.71) (end 145.415 92.71) (width 0.381) (layer F.Cu) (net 3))
 (segment (start 146.05 89.535) (end 145.415 90.17) (width 0.381) (layer F.Cu) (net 3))
 (segment (start 148.835 89.535) (end 146.05 89.535) (width 0.381) (layer F.Cu) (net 3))
 (segment (start 145.415 92.71) (end 143.265 92.71) (width 0.381) (layer F.Cu) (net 3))
 (segment (start 149.86 88.51) (end 152.4 91.05) (width 0.381) (layer F.Cu) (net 3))
 (segment (start 152.4 91.05) (end 152.4 93.218) (width 0.381) (layer F.Cu) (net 3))
 (segment (start 152.4 93.218) (end 153.797 94.615) (width 0.381) (layer F.Cu) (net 3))
 (segment (start 157.48 94.615) (end 153.797 94.615) (width 0.381) (layer F.Cu) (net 3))
 (segment (start 147.49 98.18) (end 142.8 102.87) (width 0.381) (layer F.Cu) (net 7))
 (segment (start 147.49 95.057) (end 147.49 98.18) (width 0.381) (layer F.Cu) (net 7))
 (segment (start 138.421 94.615) (end 138.43 94.624) (width 0.25) (layer F.Cu) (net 2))
 (segment (start 132.08 94.615) (end 138.421 94.615) (width 0.381) (layer F.Cu) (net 2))
 (segment (start 143.308 95.207) (end 143.265 95.25) (width 0.25) (layer F.Cu) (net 5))
 (segment (start 149.020002 95.057) (end 148.197002 94.234) (width 0.381) (layer F.Cu) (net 5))
 (segment (start 149.69 95.057) (end 149.020002 95.057) (width 0.381) (layer F.Cu) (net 5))
 (segment (start 144.281 94.234) (end 143.265 95.25) (width 0.381) (layer F.Cu) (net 5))
 (segment (start 148.197002 94.234) (end 144.281 94.234) (width 0.381) (layer F.Cu) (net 5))
 (segment (start 143.265 97.79) (end 143.265 95.25) (width 0.381) (layer F.Cu) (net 5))
 (segment (start 141.215 95.25) (end 141.215 92.71) (width 0.381) (layer F.Cu) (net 4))
 (segment (start 140.97 95.005) (end 141.215 95.25) (width 0.25) (layer F.Cu) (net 4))
 (segment (start 138.43 92.574) (end 141.079 92.574) (width 0.381) (layer F.Cu) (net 4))
 (segment (start 141.079 92.574) (end 141.215 92.71) (width 0.25) (layer F.Cu) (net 4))
 (segment (start 147.32 90.56) (end 149.86 90.56) (width 0.381) (layer F.Cu) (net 6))
 (segment (start 149.69 90.73) (end 149.86 90.56) (width 0.25) (layer F.Cu) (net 6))
 (segment (start 149.69 93.157) (end 149.69 90.73) (width 0.381) (layer F.Cu) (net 6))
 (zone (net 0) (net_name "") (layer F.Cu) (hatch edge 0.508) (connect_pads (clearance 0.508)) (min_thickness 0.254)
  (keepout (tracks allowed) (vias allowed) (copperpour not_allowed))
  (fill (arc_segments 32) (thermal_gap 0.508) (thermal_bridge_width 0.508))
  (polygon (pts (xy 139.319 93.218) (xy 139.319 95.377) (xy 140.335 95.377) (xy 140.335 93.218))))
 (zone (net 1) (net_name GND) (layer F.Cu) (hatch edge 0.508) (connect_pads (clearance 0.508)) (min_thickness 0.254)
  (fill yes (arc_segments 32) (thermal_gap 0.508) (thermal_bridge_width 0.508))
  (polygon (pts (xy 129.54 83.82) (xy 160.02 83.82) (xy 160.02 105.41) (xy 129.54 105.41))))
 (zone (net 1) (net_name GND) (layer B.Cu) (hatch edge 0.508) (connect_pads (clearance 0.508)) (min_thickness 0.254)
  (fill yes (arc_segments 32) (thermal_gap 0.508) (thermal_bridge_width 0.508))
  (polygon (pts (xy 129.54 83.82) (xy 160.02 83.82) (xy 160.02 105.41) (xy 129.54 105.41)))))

